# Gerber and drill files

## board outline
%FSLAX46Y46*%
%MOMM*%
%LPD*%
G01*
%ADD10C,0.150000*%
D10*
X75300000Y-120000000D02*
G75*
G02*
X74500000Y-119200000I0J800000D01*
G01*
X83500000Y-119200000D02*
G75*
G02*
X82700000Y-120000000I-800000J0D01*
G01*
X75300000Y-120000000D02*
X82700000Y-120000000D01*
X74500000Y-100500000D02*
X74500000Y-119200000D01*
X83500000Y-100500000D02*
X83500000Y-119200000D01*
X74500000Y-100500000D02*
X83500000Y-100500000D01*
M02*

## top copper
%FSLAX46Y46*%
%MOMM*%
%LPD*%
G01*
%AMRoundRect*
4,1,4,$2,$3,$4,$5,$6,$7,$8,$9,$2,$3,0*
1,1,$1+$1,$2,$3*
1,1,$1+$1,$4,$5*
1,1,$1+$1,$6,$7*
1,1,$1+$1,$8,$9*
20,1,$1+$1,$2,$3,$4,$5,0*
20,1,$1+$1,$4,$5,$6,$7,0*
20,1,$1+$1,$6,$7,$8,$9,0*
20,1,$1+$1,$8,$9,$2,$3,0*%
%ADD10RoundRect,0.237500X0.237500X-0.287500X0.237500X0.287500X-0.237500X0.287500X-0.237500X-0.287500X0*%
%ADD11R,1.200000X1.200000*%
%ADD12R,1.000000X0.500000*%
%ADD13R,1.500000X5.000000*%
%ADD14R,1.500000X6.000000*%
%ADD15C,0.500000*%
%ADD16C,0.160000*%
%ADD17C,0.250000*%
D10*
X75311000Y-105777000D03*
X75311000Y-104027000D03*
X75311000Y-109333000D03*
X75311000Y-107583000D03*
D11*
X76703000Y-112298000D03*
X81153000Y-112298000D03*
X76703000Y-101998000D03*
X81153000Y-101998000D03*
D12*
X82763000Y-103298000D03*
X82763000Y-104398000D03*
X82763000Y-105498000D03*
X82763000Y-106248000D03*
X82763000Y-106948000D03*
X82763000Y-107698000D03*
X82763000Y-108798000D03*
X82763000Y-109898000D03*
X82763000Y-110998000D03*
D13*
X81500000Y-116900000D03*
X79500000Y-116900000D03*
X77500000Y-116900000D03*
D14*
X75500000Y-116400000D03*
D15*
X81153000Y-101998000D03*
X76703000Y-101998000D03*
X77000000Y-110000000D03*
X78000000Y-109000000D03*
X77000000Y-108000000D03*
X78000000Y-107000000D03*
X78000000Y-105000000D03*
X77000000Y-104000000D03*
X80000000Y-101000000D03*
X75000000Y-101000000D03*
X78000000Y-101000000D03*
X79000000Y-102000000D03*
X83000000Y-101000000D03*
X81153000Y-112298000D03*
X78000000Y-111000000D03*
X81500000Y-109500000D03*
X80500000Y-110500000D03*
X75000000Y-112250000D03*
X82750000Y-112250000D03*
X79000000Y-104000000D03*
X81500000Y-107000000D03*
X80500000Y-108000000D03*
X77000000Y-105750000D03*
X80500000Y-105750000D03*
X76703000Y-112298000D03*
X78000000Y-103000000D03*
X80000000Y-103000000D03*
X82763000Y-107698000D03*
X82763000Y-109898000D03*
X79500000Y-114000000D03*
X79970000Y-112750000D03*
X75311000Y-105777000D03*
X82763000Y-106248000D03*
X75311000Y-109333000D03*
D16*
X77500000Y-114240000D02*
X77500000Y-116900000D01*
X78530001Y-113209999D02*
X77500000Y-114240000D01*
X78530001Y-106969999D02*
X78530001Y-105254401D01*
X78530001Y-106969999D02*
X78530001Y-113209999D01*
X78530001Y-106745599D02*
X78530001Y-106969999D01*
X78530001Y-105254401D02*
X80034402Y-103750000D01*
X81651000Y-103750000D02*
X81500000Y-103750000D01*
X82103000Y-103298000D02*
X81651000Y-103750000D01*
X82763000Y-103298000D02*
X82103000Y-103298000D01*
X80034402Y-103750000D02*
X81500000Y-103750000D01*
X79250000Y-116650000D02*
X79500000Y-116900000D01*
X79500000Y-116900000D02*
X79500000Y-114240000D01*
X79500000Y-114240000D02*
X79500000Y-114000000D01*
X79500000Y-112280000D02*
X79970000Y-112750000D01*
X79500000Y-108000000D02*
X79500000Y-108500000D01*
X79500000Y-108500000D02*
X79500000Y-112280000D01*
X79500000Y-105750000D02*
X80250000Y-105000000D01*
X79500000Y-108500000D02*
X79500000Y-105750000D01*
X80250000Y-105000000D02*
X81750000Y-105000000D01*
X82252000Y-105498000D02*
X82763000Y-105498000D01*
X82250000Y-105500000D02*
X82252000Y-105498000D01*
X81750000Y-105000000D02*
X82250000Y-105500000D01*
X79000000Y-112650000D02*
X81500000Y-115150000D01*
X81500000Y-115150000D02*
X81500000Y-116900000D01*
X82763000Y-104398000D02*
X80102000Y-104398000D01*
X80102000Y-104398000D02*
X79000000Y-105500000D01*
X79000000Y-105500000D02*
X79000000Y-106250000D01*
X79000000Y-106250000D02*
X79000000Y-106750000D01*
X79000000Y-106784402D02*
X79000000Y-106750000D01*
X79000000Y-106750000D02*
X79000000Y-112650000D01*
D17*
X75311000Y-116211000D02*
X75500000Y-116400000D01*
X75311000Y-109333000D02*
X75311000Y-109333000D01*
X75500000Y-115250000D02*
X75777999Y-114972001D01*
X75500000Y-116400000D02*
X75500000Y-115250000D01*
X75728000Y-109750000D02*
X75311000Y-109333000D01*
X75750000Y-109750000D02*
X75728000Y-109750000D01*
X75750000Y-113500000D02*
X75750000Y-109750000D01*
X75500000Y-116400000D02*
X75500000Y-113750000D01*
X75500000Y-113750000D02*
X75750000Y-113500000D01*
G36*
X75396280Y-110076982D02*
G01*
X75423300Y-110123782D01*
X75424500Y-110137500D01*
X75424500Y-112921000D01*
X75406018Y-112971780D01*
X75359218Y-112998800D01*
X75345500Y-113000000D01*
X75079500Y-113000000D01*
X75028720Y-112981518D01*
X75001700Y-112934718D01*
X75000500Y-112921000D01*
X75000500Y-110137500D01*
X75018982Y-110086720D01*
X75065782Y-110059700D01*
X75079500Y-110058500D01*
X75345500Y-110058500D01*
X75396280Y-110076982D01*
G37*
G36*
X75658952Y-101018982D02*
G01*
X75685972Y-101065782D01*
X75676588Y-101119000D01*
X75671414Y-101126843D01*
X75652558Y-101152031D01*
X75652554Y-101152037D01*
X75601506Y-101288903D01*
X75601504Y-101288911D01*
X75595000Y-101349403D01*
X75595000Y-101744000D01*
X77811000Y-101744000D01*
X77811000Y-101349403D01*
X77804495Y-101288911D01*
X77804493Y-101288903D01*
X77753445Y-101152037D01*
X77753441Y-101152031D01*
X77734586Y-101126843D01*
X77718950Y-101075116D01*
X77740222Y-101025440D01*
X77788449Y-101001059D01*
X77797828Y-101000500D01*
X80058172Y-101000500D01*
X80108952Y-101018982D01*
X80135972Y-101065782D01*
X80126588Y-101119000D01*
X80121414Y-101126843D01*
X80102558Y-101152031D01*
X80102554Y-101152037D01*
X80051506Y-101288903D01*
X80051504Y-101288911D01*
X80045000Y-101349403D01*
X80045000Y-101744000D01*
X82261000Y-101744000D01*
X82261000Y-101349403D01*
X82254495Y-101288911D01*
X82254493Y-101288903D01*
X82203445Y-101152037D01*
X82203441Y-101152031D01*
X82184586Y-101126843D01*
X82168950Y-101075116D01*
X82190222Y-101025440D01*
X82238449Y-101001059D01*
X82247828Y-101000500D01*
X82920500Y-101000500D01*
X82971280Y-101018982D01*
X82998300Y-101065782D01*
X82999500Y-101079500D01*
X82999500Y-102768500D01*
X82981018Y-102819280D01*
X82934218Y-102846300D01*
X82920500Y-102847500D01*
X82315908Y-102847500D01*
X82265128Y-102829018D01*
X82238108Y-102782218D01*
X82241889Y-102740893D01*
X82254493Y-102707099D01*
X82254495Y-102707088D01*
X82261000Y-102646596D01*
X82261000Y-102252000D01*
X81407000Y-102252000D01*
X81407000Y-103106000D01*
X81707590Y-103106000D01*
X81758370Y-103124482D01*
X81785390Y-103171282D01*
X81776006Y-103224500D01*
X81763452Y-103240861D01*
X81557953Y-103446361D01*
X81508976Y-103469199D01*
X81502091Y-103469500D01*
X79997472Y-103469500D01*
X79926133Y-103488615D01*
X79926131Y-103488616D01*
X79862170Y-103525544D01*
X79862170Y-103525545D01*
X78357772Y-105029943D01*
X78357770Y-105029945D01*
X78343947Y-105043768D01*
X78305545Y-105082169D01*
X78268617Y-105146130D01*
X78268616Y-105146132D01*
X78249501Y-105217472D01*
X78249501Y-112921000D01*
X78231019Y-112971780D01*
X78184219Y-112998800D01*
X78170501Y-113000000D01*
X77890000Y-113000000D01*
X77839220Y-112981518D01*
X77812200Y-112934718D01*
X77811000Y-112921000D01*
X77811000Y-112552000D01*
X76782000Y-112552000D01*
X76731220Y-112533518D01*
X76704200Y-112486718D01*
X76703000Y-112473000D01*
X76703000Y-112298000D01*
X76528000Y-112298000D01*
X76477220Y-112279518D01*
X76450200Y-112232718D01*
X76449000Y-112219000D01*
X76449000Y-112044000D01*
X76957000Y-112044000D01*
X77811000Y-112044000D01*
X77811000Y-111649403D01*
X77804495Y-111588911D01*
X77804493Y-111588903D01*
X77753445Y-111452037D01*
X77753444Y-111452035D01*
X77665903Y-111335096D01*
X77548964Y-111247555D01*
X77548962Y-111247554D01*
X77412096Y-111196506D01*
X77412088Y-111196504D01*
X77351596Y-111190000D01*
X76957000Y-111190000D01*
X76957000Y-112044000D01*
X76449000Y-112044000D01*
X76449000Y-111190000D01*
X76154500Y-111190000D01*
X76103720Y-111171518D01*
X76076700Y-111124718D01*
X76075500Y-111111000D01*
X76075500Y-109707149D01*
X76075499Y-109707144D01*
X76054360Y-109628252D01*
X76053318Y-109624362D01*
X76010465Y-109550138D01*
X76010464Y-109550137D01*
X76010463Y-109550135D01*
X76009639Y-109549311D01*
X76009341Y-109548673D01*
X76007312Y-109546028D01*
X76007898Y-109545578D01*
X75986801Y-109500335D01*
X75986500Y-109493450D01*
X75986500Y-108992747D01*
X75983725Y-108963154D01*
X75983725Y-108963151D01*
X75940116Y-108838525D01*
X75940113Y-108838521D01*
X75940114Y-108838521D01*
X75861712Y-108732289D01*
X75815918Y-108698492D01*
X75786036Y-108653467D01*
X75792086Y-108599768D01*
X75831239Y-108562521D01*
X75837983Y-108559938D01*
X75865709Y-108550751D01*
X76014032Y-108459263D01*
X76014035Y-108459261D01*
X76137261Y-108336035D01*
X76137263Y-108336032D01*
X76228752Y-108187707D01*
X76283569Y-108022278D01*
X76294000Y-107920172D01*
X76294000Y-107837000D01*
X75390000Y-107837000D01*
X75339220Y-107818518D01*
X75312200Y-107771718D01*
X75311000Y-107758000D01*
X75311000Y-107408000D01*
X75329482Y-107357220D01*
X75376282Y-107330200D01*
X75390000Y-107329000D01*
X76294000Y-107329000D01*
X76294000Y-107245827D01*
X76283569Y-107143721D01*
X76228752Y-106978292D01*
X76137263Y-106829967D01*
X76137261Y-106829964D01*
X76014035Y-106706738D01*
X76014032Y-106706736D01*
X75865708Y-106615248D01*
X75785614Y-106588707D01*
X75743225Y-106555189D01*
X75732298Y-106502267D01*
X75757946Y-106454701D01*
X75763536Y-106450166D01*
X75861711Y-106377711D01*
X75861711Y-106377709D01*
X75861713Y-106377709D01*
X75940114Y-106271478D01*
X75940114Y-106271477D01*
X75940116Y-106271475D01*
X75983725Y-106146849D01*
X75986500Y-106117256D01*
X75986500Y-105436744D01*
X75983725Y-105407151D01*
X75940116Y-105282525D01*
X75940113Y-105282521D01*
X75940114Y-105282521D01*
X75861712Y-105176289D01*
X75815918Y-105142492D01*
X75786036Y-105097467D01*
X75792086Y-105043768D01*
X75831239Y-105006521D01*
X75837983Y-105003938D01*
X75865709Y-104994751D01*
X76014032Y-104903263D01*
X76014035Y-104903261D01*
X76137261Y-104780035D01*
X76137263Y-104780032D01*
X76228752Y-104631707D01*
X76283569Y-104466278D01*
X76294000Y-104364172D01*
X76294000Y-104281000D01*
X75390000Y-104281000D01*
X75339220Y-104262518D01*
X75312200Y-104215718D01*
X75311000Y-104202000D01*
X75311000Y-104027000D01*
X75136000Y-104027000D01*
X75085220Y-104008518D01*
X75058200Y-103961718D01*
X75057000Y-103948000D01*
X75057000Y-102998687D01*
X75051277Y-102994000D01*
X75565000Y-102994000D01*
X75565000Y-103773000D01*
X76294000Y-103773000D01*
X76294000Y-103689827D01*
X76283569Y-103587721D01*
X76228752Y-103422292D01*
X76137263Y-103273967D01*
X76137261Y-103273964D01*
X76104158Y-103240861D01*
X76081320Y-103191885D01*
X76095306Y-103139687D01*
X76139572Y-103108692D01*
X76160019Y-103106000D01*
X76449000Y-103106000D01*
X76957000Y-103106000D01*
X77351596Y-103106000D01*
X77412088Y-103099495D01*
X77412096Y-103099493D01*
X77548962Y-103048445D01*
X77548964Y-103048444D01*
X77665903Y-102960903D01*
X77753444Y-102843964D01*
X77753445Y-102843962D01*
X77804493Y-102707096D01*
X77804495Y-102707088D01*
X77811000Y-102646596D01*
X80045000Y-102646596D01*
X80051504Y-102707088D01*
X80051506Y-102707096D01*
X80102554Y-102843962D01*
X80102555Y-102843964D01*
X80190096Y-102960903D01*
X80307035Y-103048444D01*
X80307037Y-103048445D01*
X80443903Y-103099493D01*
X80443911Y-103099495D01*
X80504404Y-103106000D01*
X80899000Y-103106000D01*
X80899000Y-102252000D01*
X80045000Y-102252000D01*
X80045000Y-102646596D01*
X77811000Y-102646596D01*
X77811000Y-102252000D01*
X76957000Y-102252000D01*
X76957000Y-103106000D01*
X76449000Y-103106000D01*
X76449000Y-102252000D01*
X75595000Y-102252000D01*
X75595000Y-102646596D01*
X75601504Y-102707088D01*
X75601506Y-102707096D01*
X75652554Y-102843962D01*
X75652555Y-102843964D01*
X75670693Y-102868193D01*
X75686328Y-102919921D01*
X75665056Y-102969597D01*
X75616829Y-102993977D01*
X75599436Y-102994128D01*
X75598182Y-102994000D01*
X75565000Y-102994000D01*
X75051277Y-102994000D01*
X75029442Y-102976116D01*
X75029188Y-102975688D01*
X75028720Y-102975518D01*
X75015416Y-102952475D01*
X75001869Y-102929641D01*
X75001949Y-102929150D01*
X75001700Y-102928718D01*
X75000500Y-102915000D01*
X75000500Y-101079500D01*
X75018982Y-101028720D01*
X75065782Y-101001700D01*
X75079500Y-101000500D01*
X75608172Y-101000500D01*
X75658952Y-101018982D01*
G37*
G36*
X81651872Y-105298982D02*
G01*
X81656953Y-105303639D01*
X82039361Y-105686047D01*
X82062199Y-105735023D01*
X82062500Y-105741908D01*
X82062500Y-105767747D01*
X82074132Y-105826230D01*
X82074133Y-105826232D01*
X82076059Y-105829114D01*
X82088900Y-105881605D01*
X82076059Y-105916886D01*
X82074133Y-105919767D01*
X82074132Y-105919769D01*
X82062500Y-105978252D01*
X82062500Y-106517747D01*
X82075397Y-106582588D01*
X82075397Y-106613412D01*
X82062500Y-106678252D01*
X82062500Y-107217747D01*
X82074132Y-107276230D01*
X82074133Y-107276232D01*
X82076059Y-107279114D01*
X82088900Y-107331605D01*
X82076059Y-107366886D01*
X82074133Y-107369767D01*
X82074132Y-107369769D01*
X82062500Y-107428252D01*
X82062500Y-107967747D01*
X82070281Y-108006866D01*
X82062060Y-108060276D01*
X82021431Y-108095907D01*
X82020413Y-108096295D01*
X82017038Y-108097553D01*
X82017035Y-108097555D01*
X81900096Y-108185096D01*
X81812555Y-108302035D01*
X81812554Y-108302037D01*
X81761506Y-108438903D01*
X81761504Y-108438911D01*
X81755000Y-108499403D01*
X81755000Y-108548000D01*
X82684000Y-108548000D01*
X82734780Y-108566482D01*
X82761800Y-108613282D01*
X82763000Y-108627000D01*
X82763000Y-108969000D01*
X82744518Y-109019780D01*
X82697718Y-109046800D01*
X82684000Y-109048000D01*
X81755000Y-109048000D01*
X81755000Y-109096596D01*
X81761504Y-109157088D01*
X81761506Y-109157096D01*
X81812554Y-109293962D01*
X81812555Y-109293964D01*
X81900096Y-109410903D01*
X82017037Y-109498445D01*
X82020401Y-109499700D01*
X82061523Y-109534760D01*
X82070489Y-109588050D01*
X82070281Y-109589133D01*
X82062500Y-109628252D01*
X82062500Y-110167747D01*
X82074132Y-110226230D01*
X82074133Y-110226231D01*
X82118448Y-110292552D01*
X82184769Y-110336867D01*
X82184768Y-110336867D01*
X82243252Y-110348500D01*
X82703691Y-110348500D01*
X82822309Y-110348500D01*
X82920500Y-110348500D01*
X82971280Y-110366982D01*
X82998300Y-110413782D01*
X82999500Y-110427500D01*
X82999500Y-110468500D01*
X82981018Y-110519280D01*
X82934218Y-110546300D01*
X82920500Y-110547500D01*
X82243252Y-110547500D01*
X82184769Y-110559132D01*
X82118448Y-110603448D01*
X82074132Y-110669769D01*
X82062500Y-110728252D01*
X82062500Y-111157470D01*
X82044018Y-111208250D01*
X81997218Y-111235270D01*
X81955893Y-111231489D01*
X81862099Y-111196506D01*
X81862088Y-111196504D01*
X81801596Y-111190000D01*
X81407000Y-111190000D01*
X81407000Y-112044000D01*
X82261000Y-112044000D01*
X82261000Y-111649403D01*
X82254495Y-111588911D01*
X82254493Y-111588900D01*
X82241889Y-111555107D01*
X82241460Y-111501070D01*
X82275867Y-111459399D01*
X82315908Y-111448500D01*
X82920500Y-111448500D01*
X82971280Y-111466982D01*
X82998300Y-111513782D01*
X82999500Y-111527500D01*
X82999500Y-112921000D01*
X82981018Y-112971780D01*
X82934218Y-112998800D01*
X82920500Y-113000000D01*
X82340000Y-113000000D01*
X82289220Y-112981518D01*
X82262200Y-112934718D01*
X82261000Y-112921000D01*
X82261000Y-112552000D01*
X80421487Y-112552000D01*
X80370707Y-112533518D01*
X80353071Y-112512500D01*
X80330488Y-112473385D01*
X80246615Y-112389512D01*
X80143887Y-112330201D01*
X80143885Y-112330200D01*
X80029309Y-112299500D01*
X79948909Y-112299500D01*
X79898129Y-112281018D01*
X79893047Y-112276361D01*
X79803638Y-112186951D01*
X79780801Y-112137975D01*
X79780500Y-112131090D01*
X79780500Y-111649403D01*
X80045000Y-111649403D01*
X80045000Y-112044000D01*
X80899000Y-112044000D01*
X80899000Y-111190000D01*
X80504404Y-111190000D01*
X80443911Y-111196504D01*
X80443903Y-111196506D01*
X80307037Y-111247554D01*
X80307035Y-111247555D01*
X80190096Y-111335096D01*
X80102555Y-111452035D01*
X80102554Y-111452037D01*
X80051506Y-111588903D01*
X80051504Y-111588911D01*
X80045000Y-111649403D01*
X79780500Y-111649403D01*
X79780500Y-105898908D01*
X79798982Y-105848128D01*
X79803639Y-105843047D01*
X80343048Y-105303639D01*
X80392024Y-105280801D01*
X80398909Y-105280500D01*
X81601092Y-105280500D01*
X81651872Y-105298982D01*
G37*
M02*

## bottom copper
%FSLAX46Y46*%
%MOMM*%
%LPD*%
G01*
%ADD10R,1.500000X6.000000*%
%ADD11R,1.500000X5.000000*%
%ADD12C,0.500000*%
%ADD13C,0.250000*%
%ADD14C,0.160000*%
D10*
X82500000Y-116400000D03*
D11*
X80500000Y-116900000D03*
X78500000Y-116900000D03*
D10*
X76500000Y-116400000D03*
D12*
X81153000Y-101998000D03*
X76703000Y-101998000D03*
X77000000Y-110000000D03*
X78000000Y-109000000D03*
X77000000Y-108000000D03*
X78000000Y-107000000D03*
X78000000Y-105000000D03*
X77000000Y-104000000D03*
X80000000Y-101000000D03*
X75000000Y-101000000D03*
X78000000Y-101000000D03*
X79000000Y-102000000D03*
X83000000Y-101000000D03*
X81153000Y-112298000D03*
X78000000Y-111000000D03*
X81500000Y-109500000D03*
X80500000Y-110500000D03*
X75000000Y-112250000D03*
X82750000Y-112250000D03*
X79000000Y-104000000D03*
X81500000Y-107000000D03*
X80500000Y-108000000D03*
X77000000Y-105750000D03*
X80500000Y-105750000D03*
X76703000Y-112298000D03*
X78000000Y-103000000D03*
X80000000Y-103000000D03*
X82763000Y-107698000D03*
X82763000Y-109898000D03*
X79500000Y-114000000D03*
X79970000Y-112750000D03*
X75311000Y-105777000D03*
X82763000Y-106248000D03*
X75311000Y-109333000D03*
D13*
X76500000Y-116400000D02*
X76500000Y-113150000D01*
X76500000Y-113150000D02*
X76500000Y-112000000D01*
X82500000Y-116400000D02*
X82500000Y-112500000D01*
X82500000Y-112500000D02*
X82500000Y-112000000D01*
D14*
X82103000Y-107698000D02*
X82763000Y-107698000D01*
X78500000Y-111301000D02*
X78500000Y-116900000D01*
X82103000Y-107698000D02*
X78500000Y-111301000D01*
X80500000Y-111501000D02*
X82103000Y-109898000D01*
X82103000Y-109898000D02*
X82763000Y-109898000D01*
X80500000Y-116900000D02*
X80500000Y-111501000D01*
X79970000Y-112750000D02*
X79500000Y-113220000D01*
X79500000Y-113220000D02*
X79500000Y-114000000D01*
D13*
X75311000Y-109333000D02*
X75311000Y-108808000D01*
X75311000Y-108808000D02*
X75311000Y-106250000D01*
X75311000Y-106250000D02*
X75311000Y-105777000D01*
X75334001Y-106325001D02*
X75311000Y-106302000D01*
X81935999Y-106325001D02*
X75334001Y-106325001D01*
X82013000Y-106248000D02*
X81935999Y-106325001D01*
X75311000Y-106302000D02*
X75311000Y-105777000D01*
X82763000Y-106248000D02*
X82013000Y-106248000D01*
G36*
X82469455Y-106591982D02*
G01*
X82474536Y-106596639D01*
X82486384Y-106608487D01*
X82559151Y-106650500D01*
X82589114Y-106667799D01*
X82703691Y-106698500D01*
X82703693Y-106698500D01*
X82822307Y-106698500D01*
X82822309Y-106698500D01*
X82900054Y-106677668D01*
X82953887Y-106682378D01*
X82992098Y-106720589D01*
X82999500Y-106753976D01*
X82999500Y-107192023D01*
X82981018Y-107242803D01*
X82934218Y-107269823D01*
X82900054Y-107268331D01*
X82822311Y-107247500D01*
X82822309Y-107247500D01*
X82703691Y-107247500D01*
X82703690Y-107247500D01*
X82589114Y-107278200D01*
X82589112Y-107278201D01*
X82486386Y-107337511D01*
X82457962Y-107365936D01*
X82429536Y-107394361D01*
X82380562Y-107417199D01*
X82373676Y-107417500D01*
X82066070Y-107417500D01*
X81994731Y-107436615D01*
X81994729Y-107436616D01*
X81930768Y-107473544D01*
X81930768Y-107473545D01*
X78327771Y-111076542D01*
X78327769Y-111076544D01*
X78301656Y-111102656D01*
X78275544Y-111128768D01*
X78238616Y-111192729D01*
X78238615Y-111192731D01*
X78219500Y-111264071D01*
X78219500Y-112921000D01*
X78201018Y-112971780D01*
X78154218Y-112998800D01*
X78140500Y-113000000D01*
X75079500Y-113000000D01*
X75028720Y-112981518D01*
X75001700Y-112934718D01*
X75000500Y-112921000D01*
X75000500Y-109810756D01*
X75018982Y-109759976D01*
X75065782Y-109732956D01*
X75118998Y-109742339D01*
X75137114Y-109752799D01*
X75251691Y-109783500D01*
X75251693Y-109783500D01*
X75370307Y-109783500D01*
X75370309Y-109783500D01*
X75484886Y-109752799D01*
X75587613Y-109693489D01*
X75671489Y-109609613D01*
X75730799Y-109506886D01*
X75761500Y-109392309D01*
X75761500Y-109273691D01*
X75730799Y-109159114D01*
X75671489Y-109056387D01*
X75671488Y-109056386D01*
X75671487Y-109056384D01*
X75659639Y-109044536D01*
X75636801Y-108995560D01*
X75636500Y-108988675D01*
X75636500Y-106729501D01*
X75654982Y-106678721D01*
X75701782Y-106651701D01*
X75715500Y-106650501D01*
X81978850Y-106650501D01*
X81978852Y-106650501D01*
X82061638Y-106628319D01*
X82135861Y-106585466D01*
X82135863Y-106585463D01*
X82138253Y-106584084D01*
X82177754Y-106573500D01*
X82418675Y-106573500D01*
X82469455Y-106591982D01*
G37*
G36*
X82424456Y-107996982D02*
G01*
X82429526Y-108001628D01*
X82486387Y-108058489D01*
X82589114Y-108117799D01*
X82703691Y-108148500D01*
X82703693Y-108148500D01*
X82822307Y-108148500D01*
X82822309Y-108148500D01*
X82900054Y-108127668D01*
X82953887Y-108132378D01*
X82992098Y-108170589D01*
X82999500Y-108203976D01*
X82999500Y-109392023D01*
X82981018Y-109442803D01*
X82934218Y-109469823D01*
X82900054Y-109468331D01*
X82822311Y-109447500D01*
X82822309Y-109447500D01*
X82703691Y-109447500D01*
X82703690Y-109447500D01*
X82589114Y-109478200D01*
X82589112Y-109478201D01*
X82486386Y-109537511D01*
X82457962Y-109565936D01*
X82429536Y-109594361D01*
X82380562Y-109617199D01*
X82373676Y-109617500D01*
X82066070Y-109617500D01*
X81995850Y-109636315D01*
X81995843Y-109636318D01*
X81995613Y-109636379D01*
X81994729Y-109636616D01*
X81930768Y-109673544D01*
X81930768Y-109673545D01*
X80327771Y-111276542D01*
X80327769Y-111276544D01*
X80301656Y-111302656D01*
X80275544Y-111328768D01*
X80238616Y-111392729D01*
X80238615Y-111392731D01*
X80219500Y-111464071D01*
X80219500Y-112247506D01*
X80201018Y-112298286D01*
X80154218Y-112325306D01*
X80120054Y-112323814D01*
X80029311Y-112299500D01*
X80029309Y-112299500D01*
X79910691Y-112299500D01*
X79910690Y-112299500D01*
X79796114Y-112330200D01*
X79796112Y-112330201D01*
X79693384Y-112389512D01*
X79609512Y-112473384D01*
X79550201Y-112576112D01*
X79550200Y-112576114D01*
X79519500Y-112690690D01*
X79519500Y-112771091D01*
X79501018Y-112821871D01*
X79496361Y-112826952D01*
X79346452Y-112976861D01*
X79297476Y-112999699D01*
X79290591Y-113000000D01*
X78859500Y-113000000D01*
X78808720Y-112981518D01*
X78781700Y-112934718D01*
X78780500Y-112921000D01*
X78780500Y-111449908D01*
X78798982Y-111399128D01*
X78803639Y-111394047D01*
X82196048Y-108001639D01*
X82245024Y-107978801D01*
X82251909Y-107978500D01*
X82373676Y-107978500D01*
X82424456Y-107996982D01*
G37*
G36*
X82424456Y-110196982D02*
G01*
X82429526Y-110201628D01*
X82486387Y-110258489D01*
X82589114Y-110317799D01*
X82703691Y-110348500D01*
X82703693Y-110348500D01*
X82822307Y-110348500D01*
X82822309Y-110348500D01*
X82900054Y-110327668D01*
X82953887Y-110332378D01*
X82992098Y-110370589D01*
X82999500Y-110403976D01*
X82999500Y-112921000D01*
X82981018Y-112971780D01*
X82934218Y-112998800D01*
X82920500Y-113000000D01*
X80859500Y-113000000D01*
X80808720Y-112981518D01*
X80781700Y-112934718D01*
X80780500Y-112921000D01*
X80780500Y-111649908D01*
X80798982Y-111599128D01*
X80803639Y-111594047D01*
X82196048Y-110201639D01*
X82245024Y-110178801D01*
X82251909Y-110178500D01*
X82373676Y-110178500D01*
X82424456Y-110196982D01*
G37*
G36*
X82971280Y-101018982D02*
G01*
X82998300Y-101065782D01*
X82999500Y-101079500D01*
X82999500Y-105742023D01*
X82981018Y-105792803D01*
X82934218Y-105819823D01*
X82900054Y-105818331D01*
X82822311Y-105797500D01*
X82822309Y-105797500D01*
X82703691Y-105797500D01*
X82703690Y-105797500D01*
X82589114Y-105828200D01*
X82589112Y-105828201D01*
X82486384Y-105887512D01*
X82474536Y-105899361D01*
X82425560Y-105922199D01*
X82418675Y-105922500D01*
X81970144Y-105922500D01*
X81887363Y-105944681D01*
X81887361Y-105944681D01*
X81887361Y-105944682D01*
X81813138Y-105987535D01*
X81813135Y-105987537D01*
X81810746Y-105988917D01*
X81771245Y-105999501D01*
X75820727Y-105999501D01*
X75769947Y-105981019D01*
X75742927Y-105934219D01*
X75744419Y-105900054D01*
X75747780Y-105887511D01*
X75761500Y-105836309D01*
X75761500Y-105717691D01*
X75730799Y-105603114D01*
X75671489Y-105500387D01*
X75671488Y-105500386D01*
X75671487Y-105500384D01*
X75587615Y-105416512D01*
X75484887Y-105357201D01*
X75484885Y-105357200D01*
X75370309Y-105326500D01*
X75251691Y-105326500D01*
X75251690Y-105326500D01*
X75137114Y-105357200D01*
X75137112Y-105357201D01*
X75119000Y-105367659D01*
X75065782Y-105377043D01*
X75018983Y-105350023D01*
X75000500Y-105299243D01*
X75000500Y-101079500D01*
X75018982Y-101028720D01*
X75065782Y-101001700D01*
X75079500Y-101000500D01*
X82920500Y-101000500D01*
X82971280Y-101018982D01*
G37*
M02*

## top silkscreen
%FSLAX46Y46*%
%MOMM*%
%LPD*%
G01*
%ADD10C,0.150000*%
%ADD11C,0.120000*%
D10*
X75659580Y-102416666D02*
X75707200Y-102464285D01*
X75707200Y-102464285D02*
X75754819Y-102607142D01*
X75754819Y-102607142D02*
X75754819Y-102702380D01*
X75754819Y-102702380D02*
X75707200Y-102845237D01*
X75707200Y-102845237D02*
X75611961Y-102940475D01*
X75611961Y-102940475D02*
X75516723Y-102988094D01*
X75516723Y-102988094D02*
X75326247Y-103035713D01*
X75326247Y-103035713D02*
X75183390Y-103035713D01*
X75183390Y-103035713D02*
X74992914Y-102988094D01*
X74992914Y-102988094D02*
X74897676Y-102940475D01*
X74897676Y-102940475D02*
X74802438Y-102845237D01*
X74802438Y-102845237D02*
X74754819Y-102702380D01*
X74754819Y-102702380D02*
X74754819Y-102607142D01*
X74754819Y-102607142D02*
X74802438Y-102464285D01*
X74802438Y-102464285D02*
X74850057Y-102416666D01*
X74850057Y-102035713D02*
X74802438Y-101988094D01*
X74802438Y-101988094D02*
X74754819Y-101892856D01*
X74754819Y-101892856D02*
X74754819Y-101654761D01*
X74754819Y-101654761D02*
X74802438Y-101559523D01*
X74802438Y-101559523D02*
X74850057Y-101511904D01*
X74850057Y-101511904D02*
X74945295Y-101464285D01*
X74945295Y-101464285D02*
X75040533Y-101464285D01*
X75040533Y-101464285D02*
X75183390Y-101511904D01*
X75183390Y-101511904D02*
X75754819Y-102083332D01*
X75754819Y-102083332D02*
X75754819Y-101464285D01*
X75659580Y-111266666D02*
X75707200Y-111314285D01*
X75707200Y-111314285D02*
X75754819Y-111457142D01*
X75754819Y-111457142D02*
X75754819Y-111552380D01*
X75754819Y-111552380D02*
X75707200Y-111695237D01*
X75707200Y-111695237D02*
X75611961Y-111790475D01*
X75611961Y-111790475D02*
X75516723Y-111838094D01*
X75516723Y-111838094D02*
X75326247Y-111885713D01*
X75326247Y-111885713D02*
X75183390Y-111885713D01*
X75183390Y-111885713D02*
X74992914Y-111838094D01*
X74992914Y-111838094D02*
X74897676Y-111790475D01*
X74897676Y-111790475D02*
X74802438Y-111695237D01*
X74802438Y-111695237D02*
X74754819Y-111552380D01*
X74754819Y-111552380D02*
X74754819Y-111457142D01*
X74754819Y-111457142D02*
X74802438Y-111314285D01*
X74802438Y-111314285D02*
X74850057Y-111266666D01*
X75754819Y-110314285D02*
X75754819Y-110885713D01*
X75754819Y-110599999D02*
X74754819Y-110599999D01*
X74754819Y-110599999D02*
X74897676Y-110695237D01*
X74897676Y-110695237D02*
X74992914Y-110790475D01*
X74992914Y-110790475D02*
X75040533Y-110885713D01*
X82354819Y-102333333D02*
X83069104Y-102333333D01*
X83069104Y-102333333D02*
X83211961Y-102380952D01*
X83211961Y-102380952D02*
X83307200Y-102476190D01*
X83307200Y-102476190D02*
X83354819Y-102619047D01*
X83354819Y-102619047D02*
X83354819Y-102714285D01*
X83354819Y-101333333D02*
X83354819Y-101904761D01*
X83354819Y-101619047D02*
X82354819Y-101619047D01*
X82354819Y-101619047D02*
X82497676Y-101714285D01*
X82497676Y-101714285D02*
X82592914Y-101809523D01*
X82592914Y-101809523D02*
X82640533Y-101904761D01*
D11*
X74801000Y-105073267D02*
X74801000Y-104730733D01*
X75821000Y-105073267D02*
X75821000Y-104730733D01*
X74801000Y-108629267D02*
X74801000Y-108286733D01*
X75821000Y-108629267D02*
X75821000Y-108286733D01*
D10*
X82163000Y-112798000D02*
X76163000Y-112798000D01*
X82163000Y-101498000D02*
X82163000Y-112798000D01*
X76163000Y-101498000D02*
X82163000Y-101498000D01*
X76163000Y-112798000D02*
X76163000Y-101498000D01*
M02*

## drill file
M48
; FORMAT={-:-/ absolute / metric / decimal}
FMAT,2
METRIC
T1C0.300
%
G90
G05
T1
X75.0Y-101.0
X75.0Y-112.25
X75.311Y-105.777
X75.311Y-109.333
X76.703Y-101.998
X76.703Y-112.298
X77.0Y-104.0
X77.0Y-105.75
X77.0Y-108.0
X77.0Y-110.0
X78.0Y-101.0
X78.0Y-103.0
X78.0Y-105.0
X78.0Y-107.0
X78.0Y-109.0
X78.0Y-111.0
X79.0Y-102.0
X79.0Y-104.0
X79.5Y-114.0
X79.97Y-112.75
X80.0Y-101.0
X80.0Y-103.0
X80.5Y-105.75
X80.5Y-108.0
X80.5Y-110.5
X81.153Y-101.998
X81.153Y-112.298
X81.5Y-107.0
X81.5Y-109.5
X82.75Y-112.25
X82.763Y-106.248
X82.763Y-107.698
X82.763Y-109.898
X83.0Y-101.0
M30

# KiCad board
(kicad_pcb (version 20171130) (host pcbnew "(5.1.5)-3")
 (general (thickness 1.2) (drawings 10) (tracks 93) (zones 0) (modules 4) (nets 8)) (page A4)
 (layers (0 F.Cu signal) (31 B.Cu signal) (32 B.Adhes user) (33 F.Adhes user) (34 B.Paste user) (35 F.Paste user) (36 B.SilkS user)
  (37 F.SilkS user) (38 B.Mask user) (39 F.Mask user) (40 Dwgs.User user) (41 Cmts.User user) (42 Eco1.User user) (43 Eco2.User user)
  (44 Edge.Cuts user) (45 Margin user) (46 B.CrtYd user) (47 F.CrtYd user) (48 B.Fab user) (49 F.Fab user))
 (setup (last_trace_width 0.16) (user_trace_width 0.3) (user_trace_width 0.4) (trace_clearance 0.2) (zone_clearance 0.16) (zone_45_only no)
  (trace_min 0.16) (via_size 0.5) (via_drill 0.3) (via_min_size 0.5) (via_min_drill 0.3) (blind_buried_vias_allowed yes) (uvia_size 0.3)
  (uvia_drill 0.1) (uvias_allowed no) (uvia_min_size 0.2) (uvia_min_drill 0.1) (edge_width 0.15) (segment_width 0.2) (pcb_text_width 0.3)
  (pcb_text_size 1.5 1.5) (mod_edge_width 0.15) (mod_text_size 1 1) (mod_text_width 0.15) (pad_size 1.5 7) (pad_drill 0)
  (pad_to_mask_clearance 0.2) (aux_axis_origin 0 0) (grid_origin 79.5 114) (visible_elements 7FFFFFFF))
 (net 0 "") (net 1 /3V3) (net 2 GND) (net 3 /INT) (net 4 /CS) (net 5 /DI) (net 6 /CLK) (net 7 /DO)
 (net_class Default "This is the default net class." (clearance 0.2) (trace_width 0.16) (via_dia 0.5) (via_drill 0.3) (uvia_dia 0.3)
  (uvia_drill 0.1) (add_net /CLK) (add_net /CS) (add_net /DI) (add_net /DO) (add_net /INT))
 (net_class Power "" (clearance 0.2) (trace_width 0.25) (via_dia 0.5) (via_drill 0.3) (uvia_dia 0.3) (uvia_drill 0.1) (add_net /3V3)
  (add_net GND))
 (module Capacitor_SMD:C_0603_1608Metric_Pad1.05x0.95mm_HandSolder (layer F.Cu) (at 75.311 104.902 90)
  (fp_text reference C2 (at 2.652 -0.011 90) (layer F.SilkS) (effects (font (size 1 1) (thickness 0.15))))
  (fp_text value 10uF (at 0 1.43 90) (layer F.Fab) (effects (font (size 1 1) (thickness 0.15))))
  (fp_line (start -0.171267 -0.51) (end 0.171267 -0.51) (layer F.SilkS) (width 0.12))
  (fp_line (start -0.171267 0.51) (end 0.171267 0.51) (layer F.SilkS) (width 0.12))
  (pad 1 smd roundrect (at -0.875 0 90) (size 1.05 0.95) (layers F.Cu F.Paste F.Mask) (roundrect_rratio 0.25) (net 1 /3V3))
  (pad 2 smd roundrect (at 0.875 0 90) (size 1.05 0.95) (layers F.Cu F.Paste F.Mask) (roundrect_rratio 0.25) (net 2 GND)))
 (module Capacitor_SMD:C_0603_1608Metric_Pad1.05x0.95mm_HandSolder (layer F.Cu) (at 75.311 108.458 90)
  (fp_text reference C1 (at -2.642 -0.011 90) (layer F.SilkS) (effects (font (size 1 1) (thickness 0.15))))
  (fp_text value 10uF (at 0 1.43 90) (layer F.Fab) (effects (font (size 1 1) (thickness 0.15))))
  (fp_line (start -0.171267 -0.51) (end 0.171267 -0.51) (layer F.SilkS) (width 0.12))
  (fp_line (start -0.171267 0.51) (end 0.171267 0.51) (layer F.SilkS) (width 0.12))
  (pad 1 smd roundrect (at -0.875 0 90) (size 1.05 0.95) (layers F.Cu F.Paste F.Mask) (roundrect_rratio 0.25) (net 1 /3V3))
  (pad 2 smd roundrect (at 0.875 0 90) (size 1.05 0.95) (layers F.Cu F.Paste F.Mask) (roundrect_rratio 0.25) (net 2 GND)))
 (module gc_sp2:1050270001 (layer F.Cu) (at 82.763 110.998 90)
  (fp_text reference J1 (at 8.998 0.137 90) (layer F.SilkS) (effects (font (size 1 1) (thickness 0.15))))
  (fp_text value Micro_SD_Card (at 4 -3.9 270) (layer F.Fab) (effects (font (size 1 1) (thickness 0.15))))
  (fp_line (start -1.8 -0.6) (end -1.8 -6.6) (layer F.SilkS) (width 0.15))
  (fp_line (start 9.5 -0.6) (end -1.8 -0.6) (layer F.SilkS) (width 0.15))
  (fp_line (start 9.5 -6.6) (end 9.5 -0.6) (layer F.SilkS) (width 0.15))
  (fp_line (start -1.8 -6.6) (end 9.5 -6.6) (layer F.SilkS) (width 0.15))
  (pad 9 smd rect (at -1.3 -6.06 90) (size 1.2 1.2) (layers F.Cu F.Paste F.Mask) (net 2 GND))
  (pad 9 smd rect (at -1.3 -1.61 90) (size 1.2 1.2) (layers F.Cu F.Paste F.Mask) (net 2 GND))
  (pad 9 smd rect (at 9 -6.06 90) (size 1.2 1.2) (layers F.Cu F.Paste F.Mask) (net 2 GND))
  (pad 9 smd rect (at 9 -1.61 90) (size 1.2 1.2) (layers F.Cu F.Paste F.Mask) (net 2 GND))
  (pad 1 smd rect (at 7.7 0 90) (size 0.5 1) (layers F.Cu F.Paste F.Mask) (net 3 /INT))
  (pad 2 smd rect (at 6.6 0 90) (size 0.5 1) (layers F.Cu F.Paste F.Mask) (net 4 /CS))
  (pad 3 smd rect (at 5.5 0 90) (size 0.5 1) (layers F.Cu F.Paste F.Mask) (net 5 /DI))
  (pad 4 smd rect (at 4.75 0 90) (size 0.5 1) (layers F.Cu F.Paste F.Mask) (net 1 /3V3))
  (pad "" smd rect (at 4.05 0 90) (size 0.5 1) (layers F.Cu F.Paste F.Mask))
  (pad 5 smd rect (at 3.3 0 90) (size 0.5 1) (layers F.Cu F.Paste F.Mask) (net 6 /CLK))
  (pad 6 smd rect (at 2.2 0 90) (size 0.5 1) (layers F.Cu F.Paste F.Mask) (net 2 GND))
  (pad 7 smd rect (at 1.1 0 90) (size 0.5 1) (layers F.Cu F.Paste F.Mask) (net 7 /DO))
  (pad 8 smd rect (at 0 0 90) (size 0.5 1) (layers F.Cu F.Paste F.Mask)))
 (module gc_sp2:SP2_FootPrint (layer F.Cu) (at 75.5 116.4)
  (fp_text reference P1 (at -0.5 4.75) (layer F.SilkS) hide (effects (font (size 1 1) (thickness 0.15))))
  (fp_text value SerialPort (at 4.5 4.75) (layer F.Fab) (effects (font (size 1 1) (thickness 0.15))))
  (pad 8 smd rect (at 7 0) (size 1.5 6) (layers B.Cu B.Paste B.Mask) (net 2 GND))
  (pad 7 smd rect (at 6 0.5) (size 1.5 5) (layers F.Cu F.Paste F.Mask) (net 4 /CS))
  (pad 6 smd rect (at 5 0.5) (size 1.5 5) (layers B.Cu B.Paste B.Mask) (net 7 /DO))
  (pad 5 smd rect (at 4 0.5) (size 1.5 5) (layers F.Cu F.Paste F.Mask) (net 5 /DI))
  (pad 4 smd rect (at 3 0.5) (size 1.5 5) (layers B.Cu B.Adhes B.Mask) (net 6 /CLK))
  (pad 3 smd rect (at 2 0.5) (size 1.5 5) (layers F.Cu F.Paste F.Mask) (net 3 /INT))
  (pad 2 smd rect (at 1 0) (size 1.5 6) (layers B.Cu B.Paste B.Mask) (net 2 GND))
  (pad 1 smd rect (at 0 0) (size 1.5 6) (layers F.Cu F.Paste F.Mask) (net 1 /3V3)))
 (gr_arc (start 75.3 119.2) (end 74.5 119.2) (angle -90) (layer Edge.Cuts) (width 0.15))
 (gr_arc (start 82.7 119.2) (end 83.5 119.2) (angle 90) (layer Edge.Cuts) (width 0.15))
 (gr_line (start 75.3 120) (end 82.7 120) (layer Edge.Cuts) (width 0.15))
 (gr_line (start 74.5 100.5) (end 74.5 119.2) (layer Edge.Cuts) (width 0.15))
 (gr_line (start 83.5 100.5) (end 83.5 119.2) (layer Edge.Cuts) (width 0.15))
 (gr_line (start 74.5 100.5) (end 83.5 100.5) (layer Edge.Cuts) (width 0.15))
 (via (at 81.153 101.998) (size 0.5) (drill 0.3) (layers F.Cu B.Cu) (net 2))
 (via (at 76.703 101.998) (size 0.5) (drill 0.3) (layers F.Cu B.Cu) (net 2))
 (segment (start 76.5 116.4) (end 76.5 113.15) (width 0.25) (layer B.Cu) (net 2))
 (segment (start 76.5 113.15) (end 76.5 112) (width 0.25) (layer B.Cu) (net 2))
 (segment (start 82.5 116.4) (end 82.5 112.5) (width 0.25) (layer B.Cu) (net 2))
 (segment (start 82.5 112.5) (end 82.5 112) (width 0.25) (layer B.Cu) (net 2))
 (via (at 77 110) (size 0.5) (drill 0.3) (layers F.Cu B.Cu) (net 2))
 (via (at 78 109) (size 0.5) (drill 0.3) (layers F.Cu B.Cu) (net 2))
 (via (at 77 108) (size 0.5) (drill 0.3) (layers F.Cu B.Cu) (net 2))
 (via (at 78 107) (size 0.5) (drill 0.3) (layers F.Cu B.Cu) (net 2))
 (via (at 78 105) (size 0.5) (drill 0.3) (layers F.Cu B.Cu) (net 2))
 (via (at 77 104) (size 0.5) (drill 0.3) (layers F.Cu B.Cu) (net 2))
 (via (at 80 101) (size 0.5) (drill 0.3) (layers F.Cu B.Cu) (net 2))
 (via (at 75 101) (size 0.5) (drill 0.3) (layers F.Cu B.Cu) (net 2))
 (via (at 78 101) (size 0.5) (drill 0.3) (layers F.Cu B.Cu) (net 2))
 (via (at 79 102) (size 0.5) (drill 0.3) (layers F.Cu B.Cu) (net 2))
 (via (at 83 101) (size 0.5) (drill 0.3) (layers F.Cu B.Cu) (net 2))
 (via (at 81.153 112.298) (size 0.5) (drill 0.3) (layers F.Cu B.Cu) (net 2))
 (via (at 78 111) (size 0.5) (drill 0.3) (layers F.Cu B.Cu) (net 2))
 (via (at 81.5 109.5) (size 0.5) (drill 0.3) (layers F.Cu B.Cu) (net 2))
 (via (at 80.5 110.5) (size 0.5) (drill 0.3) (layers F.Cu B.Cu) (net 2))
 (via (at 75 112.25) (size 0.5) (drill 0.3) (layers F.Cu B.Cu) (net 2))
 (via (at 82.75 112.25) (size 0.5) (drill 0.3) (layers F.Cu B.Cu) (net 2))
 (via (at 79 104) (size 0.5) (drill 0.3) (layers F.Cu B.Cu) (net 2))
 (via (at 81.5 107) (size 0.5) (drill 0.3) (layers F.Cu B.Cu) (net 2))
 (via (at 80.5 108) (size 0.5) (drill 0.3) (layers F.Cu B.Cu) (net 2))
 (via (at 77 105.75) (size 0.5) (drill 0.3) (layers F.Cu B.Cu) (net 2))
 (via (at 80.5 105.75) (size 0.5) (drill 0.3) (layers F.Cu B.Cu) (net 2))
 (via (at 76.703 112.298) (size 0.5) (drill 0.3) (layers F.Cu B.Cu) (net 2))
 (via (at 78 103) (size 0.5) (drill 0.3) (layers F.Cu B.Cu) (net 2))
 (via (at 80 103) (size 0.5) (drill 0.3) (layers F.Cu B.Cu) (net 2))
 (segment (start 77.5 114.24) (end 77.5 116.9) (width 0.16) (layer F.Cu) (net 3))
 (segment (start 78.530001 113.209999) (end 77.5 114.24) (width 0.16) (layer F.Cu) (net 3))
 (segment (start 78.530001 106.969999) (end 78.530001 105.254401) (width 0.16) (layer F.Cu) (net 3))
 (segment (start 78.530001 106.969999) (end 78.530001 113.209999) (width 0.16) (layer F.Cu) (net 3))
 (segment (start 78.530001 106.745599) (end 78.530001 106.969999) (width 0.16) (layer F.Cu) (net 3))
 (segment (start 78.530001 105.254401) (end 80.034402 103.75) (width 0.16) (layer F.Cu) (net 3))
 (segment (start 81.651 103.75) (end 81.5 103.75) (width 0.16) (layer F.Cu) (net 3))
 (segment (start 82.103 103.298) (end 81.651 103.75) (width 0.16) (layer F.Cu) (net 3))
 (segment (start 82.763 103.298) (end 82.103 103.298) (width 0.16) (layer F.Cu) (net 3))
 (segment (start 80.034402 103.75) (end 81.5 103.75) (width 0.16) (layer F.Cu) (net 3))
 (via (at 82.763 107.698) (size 0.5) (drill 0.3) (layers F.Cu B.Cu) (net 6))
 (segment (start 82.103 107.698) (end 82.763 107.698) (width 0.16) (layer B.Cu) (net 6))
 (segment (start 78.5 111.301) (end 78.5 116.9) (width 0.16) (layer B.Cu) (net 6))
 (segment (start 82.103 107.698) (end 78.5 111.301) (width 0.16) (layer B.Cu) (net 6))
 (via (at 82.763 109.898) (size 0.5) (drill 0.3) (layers F.Cu B.Cu) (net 7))
 (segment (start 80.5 111.501) (end 82.103 109.898) (width 0.16) (layer B.Cu) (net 7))
 (segment (start 82.103 109.898) (end 82.763 109.898) (width 0.16) (layer B.Cu) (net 7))
 (segment (start 80.5 116.9) (end 80.5 111.501) (width 0.16) (layer B.Cu) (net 7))
 (segment (start 79.25 116.65) (end 79.5 116.9) (width 0.16) (layer F.Cu) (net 5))
 (via (at 79.5 114) (size 0.5) (drill 0.3) (layers F.Cu B.Cu) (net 5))
 (segment (start 79.5 116.9) (end 79.5 114.24) (width 0.16) (layer F.Cu) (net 5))
 (segment (start 79.5 114.24) (end 79.5 114) (width 0.16) (layer F.Cu) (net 5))
 (via (at 79.97 112.75) (size 0.5) (drill 0.3) (layers F.Cu B.Cu) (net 5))
 (segment (start 79.5 112.28) (end 79.97 112.75) (width 0.16) (layer F.Cu) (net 5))
 (segment (start 79.97 112.75) (end 79.5 113.22) (width 0.16) (layer B.Cu) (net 5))
 (segment (start 79.5 113.22) (end 79.5 114) (width 0.16) (layer B.Cu) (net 5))
 (segment (start 79.5 108) (end 79.5 108.5) (width 0.16) (layer F.Cu) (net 5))
 (segment (start 79.5 108.5) (end 79.5 112.28) (width 0.16) (layer F.Cu) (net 5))
 (segment (start 79.5 105.75) (end 80.25 105) (width 0.16) (layer F.Cu) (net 5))
 (segment (start 79.5 108.5) (end 79.5 105.75) (width 0.16) (layer F.Cu) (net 5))
 (segment (start 80.25 105) (end 81.75 105) (width 0.16) (layer F.Cu) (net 5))
 (segment (start 82.252 105.498) (end 82.763 105.498) (width 0.16) (layer F.Cu) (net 5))
 (segment (start 82.25 105.5) (end 82.252 105.498) (width 0.16) (layer F.Cu) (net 5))
 (segment (start 81.75 105) (end 82.25 105.5) (width 0.16) (layer F.Cu) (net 5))
 (segment (start 79 112.65) (end 81.5 115.15) (width 0.16) (layer F.Cu) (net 4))
 (segment (start 81.5 115.15) (end 81.5 116.9) (width 0.16) (layer F.Cu) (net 4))
 (segment (start 82.763 104.398) (end 80.102 104.398) (width 0.16) (layer F.Cu) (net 4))
 (segment (start 80.102 104.398) (end 79 105.5) (width 0.16) (layer F.Cu) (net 4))
 (segment (start 79 105.5) (end 79 106.25) (width 0.16) (layer F.Cu) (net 4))
 (segment (start 79 106.25) (end 79 106.75) (width 0.16) (layer F.Cu) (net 4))
 (segment (start 79 106.784402) (end 79 106.75) (width 0.16) (layer F.Cu) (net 4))
 (segment (start 79 106.75) (end 79 112.65) (width 0.16) (layer F.Cu) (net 4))
 (via (at 75.311 105.777) (size 0.5) (drill 0.3) (layers F.Cu B.Cu) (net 1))
 (via (at 82.763 106.248) (size 0.5) (drill 0.3) (layers F.Cu B.Cu) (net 1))
 (segment (start 75.311 116.211) (end 75.5 116.4) (width 0.25) (layer F.Cu) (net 1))
 (segment (start 75.311 109.333) (end 75.311 109.333) (width 0.25) (layer F.Cu) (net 1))
 (via (at 75.311 109.333) (size 0.5) (drill 0.3) (layers F.Cu B.Cu) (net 1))
 (segment (start 75.311 109.333) (end 75.311 108.808) (width 0.25) (layer B.Cu) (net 1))
 (segment (start 75.311 108.808) (end 75.311 106.25) (width 0.25) (layer B.Cu) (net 1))
 (segment (start 75.311 106.25) (end 75.311 105.777) (width 0.25) (layer B.Cu) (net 1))
 (segment (start 75.334001 106.325001) (end 75.311 106.302) (width 0.25) (layer B.Cu) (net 1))
 (segment (start 81.935999 106.325001) (end 75.334001 106.325001) (width 0.25) (layer B.Cu) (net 1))
 (segment (start 82.013 106.248) (end 81.935999 106.325001) (width 0.25) (layer B.Cu) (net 1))
 (segment (start 75.311 106.302) (end 75.311 105.777) (width 0.25) (layer B.Cu) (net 1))
 (segment (start 82.763 106.248) (end 82.013 106.248) (width 0.25) (layer B.Cu) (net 1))
 (segment (start 75.5 115.25) (end 75.777999 114.972001) (width 0.25) (layer F.Cu) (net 1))
 (segment (start 75.5 116.4) (end 75.5 115.25) (width 0.25) (layer F.Cu) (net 1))
 (segment (start 75.728 109.75) (end 75.311 109.333) (width 0.25) (layer F.Cu) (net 1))
 (segment (start 75.75 109.75) (end 75.728 109.75) (width 0.25) (layer F.Cu) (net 1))
 (segment (start 75.75 113.5) (end 75.75 109.75) (width 0.25) (layer F.Cu) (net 1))
 (segment (start 75.5 116.4) (end 75.5 113.75) (width 0.25) (layer F.Cu) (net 1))
 (segment (start 75.5 113.75) (end 75.75 113.5) (width 0.25) (layer F.Cu) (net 1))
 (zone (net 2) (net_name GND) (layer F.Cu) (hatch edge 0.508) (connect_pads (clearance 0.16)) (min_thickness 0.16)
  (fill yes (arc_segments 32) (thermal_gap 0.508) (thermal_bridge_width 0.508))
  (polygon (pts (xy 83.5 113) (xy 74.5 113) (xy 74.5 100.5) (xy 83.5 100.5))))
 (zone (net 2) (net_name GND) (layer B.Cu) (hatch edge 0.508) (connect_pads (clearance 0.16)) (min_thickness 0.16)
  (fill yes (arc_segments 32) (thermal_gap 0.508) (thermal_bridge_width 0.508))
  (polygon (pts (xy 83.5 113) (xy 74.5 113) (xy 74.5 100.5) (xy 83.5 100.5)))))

